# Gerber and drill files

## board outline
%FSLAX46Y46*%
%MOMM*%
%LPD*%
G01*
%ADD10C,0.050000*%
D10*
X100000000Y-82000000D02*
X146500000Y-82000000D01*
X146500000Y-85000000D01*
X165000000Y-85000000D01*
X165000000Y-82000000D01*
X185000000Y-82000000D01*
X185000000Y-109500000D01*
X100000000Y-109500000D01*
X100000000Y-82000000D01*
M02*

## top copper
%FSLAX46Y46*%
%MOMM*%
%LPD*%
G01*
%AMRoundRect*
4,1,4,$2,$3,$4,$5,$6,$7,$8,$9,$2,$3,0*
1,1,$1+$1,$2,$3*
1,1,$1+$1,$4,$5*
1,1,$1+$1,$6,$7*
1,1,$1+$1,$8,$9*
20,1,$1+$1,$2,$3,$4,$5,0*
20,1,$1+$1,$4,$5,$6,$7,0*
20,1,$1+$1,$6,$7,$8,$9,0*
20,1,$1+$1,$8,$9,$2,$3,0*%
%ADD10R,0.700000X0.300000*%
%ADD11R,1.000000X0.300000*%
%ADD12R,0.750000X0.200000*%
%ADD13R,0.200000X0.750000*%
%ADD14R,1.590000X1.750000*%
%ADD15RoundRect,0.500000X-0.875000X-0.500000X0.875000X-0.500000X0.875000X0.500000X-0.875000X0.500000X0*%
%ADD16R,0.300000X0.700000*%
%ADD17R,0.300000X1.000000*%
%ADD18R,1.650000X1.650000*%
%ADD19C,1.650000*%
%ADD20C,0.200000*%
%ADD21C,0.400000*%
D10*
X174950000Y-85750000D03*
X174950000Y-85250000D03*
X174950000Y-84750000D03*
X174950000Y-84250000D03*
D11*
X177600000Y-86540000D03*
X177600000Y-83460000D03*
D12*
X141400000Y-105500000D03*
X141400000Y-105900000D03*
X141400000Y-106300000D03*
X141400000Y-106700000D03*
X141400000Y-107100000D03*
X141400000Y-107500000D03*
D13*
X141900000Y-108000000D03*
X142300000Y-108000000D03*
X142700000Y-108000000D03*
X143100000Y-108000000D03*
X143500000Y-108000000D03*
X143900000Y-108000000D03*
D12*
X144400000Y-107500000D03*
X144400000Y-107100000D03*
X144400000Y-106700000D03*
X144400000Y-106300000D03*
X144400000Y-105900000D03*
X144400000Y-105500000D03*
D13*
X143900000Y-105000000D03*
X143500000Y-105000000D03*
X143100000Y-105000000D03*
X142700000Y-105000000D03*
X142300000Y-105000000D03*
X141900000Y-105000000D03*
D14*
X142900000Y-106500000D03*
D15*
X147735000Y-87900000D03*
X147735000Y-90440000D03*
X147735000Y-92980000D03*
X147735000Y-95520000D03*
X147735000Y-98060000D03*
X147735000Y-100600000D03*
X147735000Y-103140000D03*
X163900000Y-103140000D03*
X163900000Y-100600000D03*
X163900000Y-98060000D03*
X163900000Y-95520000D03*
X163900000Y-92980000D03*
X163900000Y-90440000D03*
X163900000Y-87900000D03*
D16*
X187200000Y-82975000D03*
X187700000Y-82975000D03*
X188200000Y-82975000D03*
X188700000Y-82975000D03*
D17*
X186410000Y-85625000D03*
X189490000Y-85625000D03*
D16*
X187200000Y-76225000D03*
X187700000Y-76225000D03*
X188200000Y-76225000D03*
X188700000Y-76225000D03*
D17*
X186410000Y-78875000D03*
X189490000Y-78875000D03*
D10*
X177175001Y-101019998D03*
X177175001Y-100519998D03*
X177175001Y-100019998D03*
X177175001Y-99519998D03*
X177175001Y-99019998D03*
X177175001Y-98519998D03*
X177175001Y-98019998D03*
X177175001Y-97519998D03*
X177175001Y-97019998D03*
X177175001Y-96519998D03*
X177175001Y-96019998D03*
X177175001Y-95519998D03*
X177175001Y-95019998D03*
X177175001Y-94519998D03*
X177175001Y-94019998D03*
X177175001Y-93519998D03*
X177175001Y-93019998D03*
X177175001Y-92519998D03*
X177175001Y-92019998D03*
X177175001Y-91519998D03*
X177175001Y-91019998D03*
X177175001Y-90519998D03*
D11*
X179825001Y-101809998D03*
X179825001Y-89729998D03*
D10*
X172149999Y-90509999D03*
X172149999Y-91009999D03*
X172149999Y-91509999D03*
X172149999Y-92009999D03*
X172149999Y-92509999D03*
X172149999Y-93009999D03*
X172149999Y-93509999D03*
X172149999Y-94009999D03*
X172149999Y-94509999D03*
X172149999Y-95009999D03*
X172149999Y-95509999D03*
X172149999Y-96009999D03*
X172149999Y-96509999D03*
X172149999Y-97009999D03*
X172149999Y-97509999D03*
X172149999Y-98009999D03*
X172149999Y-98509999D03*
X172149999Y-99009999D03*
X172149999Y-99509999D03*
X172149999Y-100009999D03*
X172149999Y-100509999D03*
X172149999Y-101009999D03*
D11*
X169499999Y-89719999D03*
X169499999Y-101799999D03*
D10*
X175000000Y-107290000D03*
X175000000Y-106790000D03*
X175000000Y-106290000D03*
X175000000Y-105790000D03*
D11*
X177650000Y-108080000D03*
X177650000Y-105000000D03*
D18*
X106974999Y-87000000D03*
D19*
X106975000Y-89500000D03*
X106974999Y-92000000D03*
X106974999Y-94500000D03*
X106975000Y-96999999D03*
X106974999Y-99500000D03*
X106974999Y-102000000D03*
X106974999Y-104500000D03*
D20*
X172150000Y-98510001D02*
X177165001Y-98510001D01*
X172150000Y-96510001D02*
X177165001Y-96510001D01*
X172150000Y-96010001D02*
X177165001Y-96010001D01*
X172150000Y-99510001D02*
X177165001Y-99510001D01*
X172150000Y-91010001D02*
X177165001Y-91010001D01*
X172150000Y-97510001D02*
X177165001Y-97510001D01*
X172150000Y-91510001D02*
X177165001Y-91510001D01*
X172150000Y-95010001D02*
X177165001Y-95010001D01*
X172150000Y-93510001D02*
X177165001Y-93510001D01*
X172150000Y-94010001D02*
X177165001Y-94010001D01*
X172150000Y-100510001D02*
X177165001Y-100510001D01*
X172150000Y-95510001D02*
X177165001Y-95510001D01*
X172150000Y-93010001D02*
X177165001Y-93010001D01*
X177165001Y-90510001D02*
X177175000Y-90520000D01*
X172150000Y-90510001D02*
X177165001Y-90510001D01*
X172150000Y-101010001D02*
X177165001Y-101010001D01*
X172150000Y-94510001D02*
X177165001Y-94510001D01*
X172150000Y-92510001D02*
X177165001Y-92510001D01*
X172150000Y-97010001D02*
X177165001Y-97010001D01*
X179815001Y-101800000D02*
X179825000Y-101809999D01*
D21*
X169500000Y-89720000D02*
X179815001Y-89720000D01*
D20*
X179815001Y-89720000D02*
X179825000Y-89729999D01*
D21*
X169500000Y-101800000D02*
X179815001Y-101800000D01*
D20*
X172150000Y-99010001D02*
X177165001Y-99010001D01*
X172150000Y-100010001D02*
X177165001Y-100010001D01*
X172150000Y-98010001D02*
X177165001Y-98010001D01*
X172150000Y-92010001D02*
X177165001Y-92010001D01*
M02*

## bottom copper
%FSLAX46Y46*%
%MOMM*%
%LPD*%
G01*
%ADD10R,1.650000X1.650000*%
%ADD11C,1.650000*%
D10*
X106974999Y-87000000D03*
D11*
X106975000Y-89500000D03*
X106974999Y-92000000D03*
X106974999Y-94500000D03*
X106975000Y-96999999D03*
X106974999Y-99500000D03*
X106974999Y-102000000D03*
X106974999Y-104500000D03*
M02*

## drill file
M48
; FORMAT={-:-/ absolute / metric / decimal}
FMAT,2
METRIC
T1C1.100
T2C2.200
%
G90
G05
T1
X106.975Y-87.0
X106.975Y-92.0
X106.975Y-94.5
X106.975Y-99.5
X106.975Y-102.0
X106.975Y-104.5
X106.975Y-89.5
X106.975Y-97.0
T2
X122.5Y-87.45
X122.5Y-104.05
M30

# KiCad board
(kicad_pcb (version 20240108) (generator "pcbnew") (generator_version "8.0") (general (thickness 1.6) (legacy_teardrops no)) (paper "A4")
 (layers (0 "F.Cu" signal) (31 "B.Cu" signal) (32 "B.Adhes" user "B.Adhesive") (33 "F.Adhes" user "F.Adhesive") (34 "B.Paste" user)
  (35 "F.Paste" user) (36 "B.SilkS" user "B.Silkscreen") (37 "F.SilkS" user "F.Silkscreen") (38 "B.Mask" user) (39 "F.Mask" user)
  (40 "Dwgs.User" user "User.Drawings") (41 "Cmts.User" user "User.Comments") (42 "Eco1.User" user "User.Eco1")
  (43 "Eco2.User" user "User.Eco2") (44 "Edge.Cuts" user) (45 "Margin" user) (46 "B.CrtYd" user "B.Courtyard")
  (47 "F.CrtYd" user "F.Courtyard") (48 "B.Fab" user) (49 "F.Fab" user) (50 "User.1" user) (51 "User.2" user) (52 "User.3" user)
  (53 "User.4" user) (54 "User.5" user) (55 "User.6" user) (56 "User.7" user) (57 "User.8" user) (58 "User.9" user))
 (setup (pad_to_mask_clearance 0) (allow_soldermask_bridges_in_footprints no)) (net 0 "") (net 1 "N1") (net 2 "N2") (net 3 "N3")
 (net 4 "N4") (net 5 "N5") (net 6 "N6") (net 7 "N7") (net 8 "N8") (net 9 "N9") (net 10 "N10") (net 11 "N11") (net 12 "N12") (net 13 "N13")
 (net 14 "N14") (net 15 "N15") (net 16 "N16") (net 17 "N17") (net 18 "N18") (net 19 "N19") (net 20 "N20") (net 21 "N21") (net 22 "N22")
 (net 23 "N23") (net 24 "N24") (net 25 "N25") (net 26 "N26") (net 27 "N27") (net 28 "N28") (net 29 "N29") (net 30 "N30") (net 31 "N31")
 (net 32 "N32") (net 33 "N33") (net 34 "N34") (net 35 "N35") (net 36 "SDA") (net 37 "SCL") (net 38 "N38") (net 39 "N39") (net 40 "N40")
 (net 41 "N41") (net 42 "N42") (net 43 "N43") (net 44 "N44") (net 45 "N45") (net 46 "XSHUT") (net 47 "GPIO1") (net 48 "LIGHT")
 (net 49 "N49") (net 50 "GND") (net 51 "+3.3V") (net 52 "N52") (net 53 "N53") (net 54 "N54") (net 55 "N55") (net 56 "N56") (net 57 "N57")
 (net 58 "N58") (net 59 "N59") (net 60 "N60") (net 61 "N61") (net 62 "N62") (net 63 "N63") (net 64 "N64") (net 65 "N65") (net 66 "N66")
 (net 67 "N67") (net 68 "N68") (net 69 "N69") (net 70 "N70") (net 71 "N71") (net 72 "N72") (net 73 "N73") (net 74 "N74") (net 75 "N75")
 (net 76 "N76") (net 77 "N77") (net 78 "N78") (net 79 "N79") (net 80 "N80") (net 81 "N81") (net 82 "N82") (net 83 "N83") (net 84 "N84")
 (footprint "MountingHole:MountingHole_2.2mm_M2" (layer "F.Cu") (at 122.5 104.05)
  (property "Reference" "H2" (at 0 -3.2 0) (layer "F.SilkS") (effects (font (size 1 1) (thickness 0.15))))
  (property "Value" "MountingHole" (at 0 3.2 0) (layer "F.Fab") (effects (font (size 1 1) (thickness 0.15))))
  (pad "" np_thru_hole circle (at 0 0) (size 2.2 2.2) (drill 2.2) (layers "*.Cu" "*.Mask")))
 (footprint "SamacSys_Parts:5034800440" (layer "F.Cu") (at 176.45 85 90)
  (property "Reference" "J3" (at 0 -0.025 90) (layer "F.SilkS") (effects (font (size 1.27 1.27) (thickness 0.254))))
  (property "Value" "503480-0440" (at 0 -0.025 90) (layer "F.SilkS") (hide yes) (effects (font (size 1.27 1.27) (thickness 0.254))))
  (pad "1" smd rect (at -0.75 -1.5 90) (size 0.3 0.7) (layers "F.Cu" "F.Paste" "F.Mask") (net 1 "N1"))
  (pad "2" smd rect (at -0.25 -1.5 90) (size 0.3 0.7) (layers "F.Cu" "F.Paste" "F.Mask") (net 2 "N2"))
  (pad "3" smd rect (at 0.25 -1.5 90) (size 0.3 0.7) (layers "F.Cu" "F.Paste" "F.Mask") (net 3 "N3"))
  (pad "4" smd rect (at 0.75 -1.5 90) (size 0.3 0.7) (layers "F.Cu" "F.Paste" "F.Mask") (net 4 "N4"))
  (pad "MP1" smd rect (at -1.54 1.15 90) (size 0.3 1) (layers "F.Cu" "F.Paste" "F.Mask") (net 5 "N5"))
  (pad "MP2" smd rect (at 1.54 1.15 90) (size 0.3 1) (layers "F.Cu" "F.Paste" "F.Mask") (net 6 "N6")))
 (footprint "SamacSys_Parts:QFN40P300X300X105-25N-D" (layer "F.Cu") (at 142.9 106.5)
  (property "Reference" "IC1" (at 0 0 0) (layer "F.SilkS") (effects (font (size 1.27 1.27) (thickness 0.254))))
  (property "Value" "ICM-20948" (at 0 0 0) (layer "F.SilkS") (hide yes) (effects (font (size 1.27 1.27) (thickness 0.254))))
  (pad "1" smd rect (at -1.5 -1 90) (size 0.2 0.75) (layers "F.Cu" "F.Paste" "F.Mask") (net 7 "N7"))
  (pad "2" smd rect (at -1.5 -0.6 90) (size 0.2 0.75) (layers "F.Cu" "F.Paste" "F.Mask") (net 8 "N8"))
  (pad "3" smd rect (at -1.5 -0.2 90) (size 0.2 0.75) (layers "F.Cu" "F.Paste" "F.Mask") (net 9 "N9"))
  (pad "4" smd rect (at -1.5 0.2 90) (size 0.2 0.75) (layers "F.Cu" "F.Paste" "F.Mask") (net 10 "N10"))
  (pad "5" smd rect (at -1.5 0.6 90) (size 0.2 0.75) (layers "F.Cu" "F.Paste" "F.Mask") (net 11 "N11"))
  (pad "6" smd rect (at -1.5 1 90) (size 0.2 0.75) (layers "F.Cu" "F.Paste" "F.Mask") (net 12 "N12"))
  (pad "7" smd rect (at -1 1.5) (size 0.2 0.75) (layers "F.Cu" "F.Paste" "F.Mask") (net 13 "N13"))
  (pad "8" smd rect (at -0.6 1.5) (size 0.2 0.75) (layers "F.Cu" "F.Paste" "F.Mask") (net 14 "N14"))
  (pad "9" smd rect (at -0.2 1.5) (size 0.2 0.75) (layers "F.Cu" "F.Paste" "F.Mask") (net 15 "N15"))
  (pad "10" smd rect (at 0.2 1.5) (size 0.2 0.75) (layers "F.Cu" "F.Paste" "F.Mask") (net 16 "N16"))
  (pad "11" smd rect (at 0.6 1.5) (size 0.2 0.75) (layers "F.Cu" "F.Paste" "F.Mask") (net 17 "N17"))
  (pad "12" smd rect (at 1 1.5) (size 0.2 0.75) (layers "F.Cu" "F.Paste" "F.Mask") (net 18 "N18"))
  (pad "13" smd rect (at 1.5 1 90) (size 0.2 0.75) (layers "F.Cu" "F.Paste" "F.Mask") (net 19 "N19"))
  (pad "14" smd rect (at 1.5 0.6 90) (size 0.2 0.75) (layers "F.Cu" "F.Paste" "F.Mask") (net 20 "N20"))
  (pad "15" smd rect (at 1.5 0.2 90) (size 0.2 0.75) (layers "F.Cu" "F.Paste" "F.Mask") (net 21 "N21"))
  (pad "16" smd rect (at 1.5 -0.2 90) (size 0.2 0.75) (layers "F.Cu" "F.Paste" "F.Mask") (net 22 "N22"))
  (pad "17" smd rect (at 1.5 -0.6 90) (size 0.2 0.75) (layers "F.Cu" "F.Paste" "F.Mask") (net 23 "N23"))
  (pad "18" smd rect (at 1.5 -1 90) (size 0.2 0.75) (layers "F.Cu" "F.Paste" "F.Mask") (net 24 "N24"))
  (pad "19" smd rect (at 1 -1.5) (size 0.2 0.75) (layers "F.Cu" "F.Paste" "F.Mask") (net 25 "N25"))
  (pad "20" smd rect (at 0.6 -1.5) (size 0.2 0.75) (layers "F.Cu" "F.Paste" "F.Mask") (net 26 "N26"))
  (pad "21" smd rect (at 0.2 -1.5) (size 0.2 0.75) (layers "F.Cu" "F.Paste" "F.Mask") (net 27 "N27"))
  (pad "22" smd rect (at -0.2 -1.5) (size 0.2 0.75) (layers "F.Cu" "F.Paste" "F.Mask") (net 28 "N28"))
  (pad "23" smd rect (at -0.6 -1.5) (size 0.2 0.75) (layers "F.Cu" "F.Paste" "F.Mask") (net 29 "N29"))
  (pad "24" smd rect (at -1 -1.5) (size 0.2 0.75) (layers "F.Cu" "F.Paste" "F.Mask") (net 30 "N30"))
  (pad "25" smd rect (at 0 0) (size 1.59 1.75) (layers "F.Cu" "F.Paste" "F.Mask") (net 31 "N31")))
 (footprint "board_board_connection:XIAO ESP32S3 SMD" (layer "F.Cu") (at 155.796364 95.473)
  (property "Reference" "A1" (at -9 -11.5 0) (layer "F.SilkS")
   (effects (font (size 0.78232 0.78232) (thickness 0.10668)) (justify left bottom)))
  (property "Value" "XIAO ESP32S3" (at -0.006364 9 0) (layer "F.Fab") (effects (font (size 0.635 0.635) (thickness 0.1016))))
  (pad "1" smd roundrect (at -8.061364 -7.573) (size 2.75 2) (layers "F.Cu" "F.Paste" "F.Mask") (roundrect_rratio 0.25) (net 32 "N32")
   (solder_mask_margin 0.0508) (thermal_bridge_angle 45))
  (pad "2" smd roundrect (at -8.061364 -5.033) (size 2.75 2) (layers "F.Cu" "F.Paste" "F.Mask") (roundrect_rratio 0.25) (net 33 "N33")
   (solder_mask_margin 0.0508) (thermal_bridge_angle 45))
  (pad "3" smd roundrect (at -8.061364 -2.493) (size 2.75 2) (layers "F.Cu" "F.Paste" "F.Mask") (roundrect_rratio 0.25) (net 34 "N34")
   (solder_mask_margin 0.0508) (thermal_bridge_angle 45))
  (pad "4" smd roundrect (at -8.061364 0.047) (size 2.75 2) (layers "F.Cu" "F.Paste" "F.Mask") (roundrect_rratio 0.25) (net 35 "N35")
   (solder_mask_margin 0.0508) (thermal_bridge_angle 45))
  (pad "5" smd roundrect (at -8.061364 2.587) (size 2.75 2) (layers "F.Cu" "F.Paste" "F.Mask") (roundrect_rratio 0.25) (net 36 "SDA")
   (solder_mask_margin 0.0508) (thermal_bridge_angle 45))
  (pad "6" smd roundrect (at -8.061364 5.127) (size 2.75 2) (layers "F.Cu" "F.Paste" "F.Mask") (roundrect_rratio 0.25) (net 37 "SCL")
   (solder_mask_margin 0.0508) (thermal_bridge_angle 45))
  (pad "7" smd roundrect (at -8.061364 7.667) (size 2.75 2) (layers "F.Cu" "F.Paste" "F.Mask") (roundrect_rratio 0.25) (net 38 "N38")
   (solder_mask_margin 0.0508) (thermal_bridge_angle 45))
  (pad "8" smd roundrect (at 8.103636 7.667) (size 2.75 2) (layers "F.Cu" "F.Paste" "F.Mask") (roundrect_rratio 0.25) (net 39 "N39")
   (solder_mask_margin 0.0508) (thermal_bridge_angle 45))
  (pad "9" smd roundrect (at 8.103636 5.127) (size 2.75 2) (layers "F.Cu" "F.Paste" "F.Mask") (roundrect_rratio 0.25) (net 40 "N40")
   (solder_mask_margin 0.0508) (thermal_bridge_angle 45))
  (pad "10" smd roundrect (at 8.103636 2.587) (size 2.75 2) (layers "F.Cu" "F.Paste" "F.Mask") (roundrect_rratio 0.25) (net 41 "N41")
   (solder_mask_margin 0.0508) (thermal_bridge_angle 45))
  (pad "11" smd roundrect (at 8.103636 0.047) (size 2.75 2) (layers "F.Cu" "F.Paste" "F.Mask") (roundrect_rratio 0.25) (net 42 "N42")
   (solder_mask_margin 0.0508) (thermal_bridge_angle 45))
  (pad "12" smd roundrect (at 8.103636 -2.493) (size 2.75 2) (layers "F.Cu" "F.Paste" "F.Mask") (roundrect_rratio 0.25) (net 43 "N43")
   (solder_mask_margin 0.0508) (thermal_bridge_angle 45))
  (pad "13" smd roundrect (at 8.103636 -5.033) (size 2.75 2) (layers "F.Cu" "F.Paste" "F.Mask") (roundrect_rratio 0.25) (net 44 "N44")
   (solder_mask_margin 0.0508) (thermal_bridge_angle 45))
  (pad "14" smd roundrect (at 8.103636 -7.573) (size 2.75 2) (layers "F.Cu" "F.Paste" "F.Mask") (roundrect_rratio 0.25) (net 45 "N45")
   (solder_mask_margin 0.0508) (thermal_bridge_angle 45)))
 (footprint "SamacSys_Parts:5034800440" (layer "F.Cu") (at 187.95 84.475)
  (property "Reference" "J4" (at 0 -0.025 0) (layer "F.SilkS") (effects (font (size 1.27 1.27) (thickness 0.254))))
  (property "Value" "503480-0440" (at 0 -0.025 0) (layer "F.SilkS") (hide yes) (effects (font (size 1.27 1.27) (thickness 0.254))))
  (pad "1" smd rect (at -0.75 -1.5) (size 0.3 0.7) (layers "F.Cu" "F.Paste" "F.Mask") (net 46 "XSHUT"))
  (pad "2" smd rect (at -0.25 -1.5) (size 0.3 0.7) (layers "F.Cu" "F.Paste" "F.Mask") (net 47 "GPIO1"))
  (pad "3" smd rect (at 0.25 -1.5) (size 0.3 0.7) (layers "F.Cu" "F.Paste" "F.Mask") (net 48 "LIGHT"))
  (pad "4" smd rect (at 0.75 -1.5) (size 0.3 0.7) (layers "F.Cu" "F.Paste" "F.Mask") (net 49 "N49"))
  (pad "MP1" smd rect (at -1.54 1.15) (size 0.3 1) (layers "F.Cu" "F.Paste" "F.Mask") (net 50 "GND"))
  (pad "MP2" smd rect (at 1.54 1.15) (size 0.3 1) (layers "F.Cu" "F.Paste" "F.Mask") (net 50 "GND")))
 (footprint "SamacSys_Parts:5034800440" (layer "F.Cu") (at 187.95 77.725)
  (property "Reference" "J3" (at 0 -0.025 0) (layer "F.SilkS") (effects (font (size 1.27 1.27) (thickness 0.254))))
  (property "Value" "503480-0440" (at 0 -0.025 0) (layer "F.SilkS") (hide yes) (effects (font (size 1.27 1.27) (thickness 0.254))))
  (pad "1" smd rect (at -0.75 -1.5) (size 0.3 0.7) (layers "F.Cu" "F.Paste" "F.Mask") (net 36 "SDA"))
  (pad "2" smd rect (at -0.25 -1.5) (size 0.3 0.7) (layers "F.Cu" "F.Paste" "F.Mask") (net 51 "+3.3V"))
  (pad "3" smd rect (at 0.25 -1.5) (size 0.3 0.7) (layers "F.Cu" "F.Paste" "F.Mask") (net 37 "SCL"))
  (pad "4" smd rect (at 0.75 -1.5) (size 0.3 0.7) (layers "F.Cu" "F.Paste" "F.Mask") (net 50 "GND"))
  (pad "MP1" smd rect (at -1.54 1.15) (size 0.3 1) (layers "F.Cu" "F.Paste" "F.Mask") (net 50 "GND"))
  (pad "MP2" smd rect (at 1.54 1.15) (size 0.3 1) (layers "F.Cu" "F.Paste" "F.Mask") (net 50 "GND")))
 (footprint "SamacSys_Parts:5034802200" (layer "F.Cu") (at 176.925001 95.769998 90)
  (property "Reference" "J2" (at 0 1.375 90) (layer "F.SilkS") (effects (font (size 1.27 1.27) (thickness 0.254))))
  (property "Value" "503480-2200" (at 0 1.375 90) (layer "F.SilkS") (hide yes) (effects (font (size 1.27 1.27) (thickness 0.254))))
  (pad "1" smd rect (at -5.25 0.25 90) (size 0.3 0.7) (layers "F.Cu" "F.Paste" "F.Mask") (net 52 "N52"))
  (pad "2" smd rect (at -4.75 0.25 90) (size 0.3 0.7) (layers "F.Cu" "F.Paste" "F.Mask") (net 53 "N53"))
  (pad "3" smd rect (at -4.25 0.25 90) (size 0.3 0.7) (layers "F.Cu" "F.Paste" "F.Mask") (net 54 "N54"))
  (pad "4" smd rect (at -3.75 0.25 90) (size 0.3 0.7) (layers "F.Cu" "F.Paste" "F.Mask") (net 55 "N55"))
  (pad "5" smd rect (at -3.25 0.25 90) (size 0.3 0.7) (layers "F.Cu" "F.Paste" "F.Mask") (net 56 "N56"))
  (pad "6" smd rect (at -2.75 0.25 90) (size 0.3 0.7) (layers "F.Cu" "F.Paste" "F.Mask") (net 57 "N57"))
  (pad "7" smd rect (at -2.25 0.25 90) (size 0.3 0.7) (layers "F.Cu" "F.Paste" "F.Mask") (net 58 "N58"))
  (pad "8" smd rect (at -1.75 0.25 90) (size 0.3 0.7) (layers "F.Cu" "F.Paste" "F.Mask") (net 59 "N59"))
  (pad "9" smd rect (at -1.25 0.25 90) (size 0.3 0.7) (layers "F.Cu" "F.Paste" "F.Mask") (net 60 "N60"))
  (pad "10" smd rect (at -0.75 0.25 90) (size 0.3 0.7) (layers "F.Cu" "F.Paste" "F.Mask") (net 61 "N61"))
  (pad "11" smd rect (at -0.25 0.25 90) (size 0.3 0.7) (layers "F.Cu" "F.Paste" "F.Mask") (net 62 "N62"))
  (pad "12" smd rect (at 0.25 0.25 90) (size 0.3 0.7) (layers "F.Cu" "F.Paste" "F.Mask") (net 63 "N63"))
  (pad "13" smd rect (at 0.75 0.25 90) (size 0.3 0.7) (layers "F.Cu" "F.Paste" "F.Mask") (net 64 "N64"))
  (pad "14" smd rect (at 1.25 0.25 90) (size 0.3 0.7) (layers "F.Cu" "F.Paste" "F.Mask") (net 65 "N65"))
  (pad "15" smd rect (at 1.75 0.25 90) (size 0.3 0.7) (layers "F.Cu" "F.Paste" "F.Mask") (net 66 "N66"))
  (pad "16" smd rect (at 2.25 0.25 90) (size 0.3 0.7) (layers "F.Cu" "F.Paste" "F.Mask") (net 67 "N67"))
  (pad "17" smd rect (at 2.75 0.25 90) (size 0.3 0.7) (layers "F.Cu" "F.Paste" "F.Mask") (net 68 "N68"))
  (pad "18" smd rect (at 3.25 0.25 90) (size 0.3 0.7) (layers "F.Cu" "F.Paste" "F.Mask") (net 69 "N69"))
  (pad "19" smd rect (at 3.75 0.25 90) (size 0.3 0.7) (layers "F.Cu" "F.Paste" "F.Mask") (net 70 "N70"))
  (pad "20" smd rect (at 4.25 0.25 90) (size 0.3 0.7) (layers "F.Cu" "F.Paste" "F.Mask") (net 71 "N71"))
  (pad "21" smd rect (at 4.75 0.25 90) (size 0.3 0.7) (layers "F.Cu" "F.Paste" "F.Mask") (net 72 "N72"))
  (pad "22" smd rect (at 5.25 0.25 90) (size 0.3 0.7) (layers "F.Cu" "F.Paste" "F.Mask") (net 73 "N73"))
  (pad "MP1" smd rect (at -6.04 2.9 90) (size 0.3 1) (layers "F.Cu" "F.Paste" "F.Mask") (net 50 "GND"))
  (pad "MP2" smd rect (at 6.04 2.9 90) (size 0.3 1) (layers "F.Cu" "F.Paste" "F.Mask") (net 50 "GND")))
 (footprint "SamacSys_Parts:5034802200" (layer "F.Cu") (at 172.399999 95.759999 -90)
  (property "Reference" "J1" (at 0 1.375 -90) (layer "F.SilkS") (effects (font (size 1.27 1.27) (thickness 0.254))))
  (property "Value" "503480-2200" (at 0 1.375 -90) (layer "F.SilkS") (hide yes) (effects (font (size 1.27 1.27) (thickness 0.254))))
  (pad "1" smd rect (at -5.25 0.25 270) (size 0.3 0.7) (layers "F.Cu" "F.Paste" "F.Mask") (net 73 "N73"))
  (pad "2" smd rect (at -4.75 0.25 270) (size 0.3 0.7) (layers "F.Cu" "F.Paste" "F.Mask") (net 72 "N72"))
  (pad "3" smd rect (at -4.25 0.25 270) (size 0.3 0.7) (layers "F.Cu" "F.Paste" "F.Mask") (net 71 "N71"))
  (pad "4" smd rect (at -3.75 0.25 270) (size 0.3 0.7) (layers "F.Cu" "F.Paste" "F.Mask") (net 70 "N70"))
  (pad "5" smd rect (at -3.25 0.25 270) (size 0.3 0.7) (layers "F.Cu" "F.Paste" "F.Mask") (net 69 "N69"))
  (pad "6" smd rect (at -2.75 0.25 270) (size 0.3 0.7) (layers "F.Cu" "F.Paste" "F.Mask") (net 68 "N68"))
  (pad "7" smd rect (at -2.25 0.25 270) (size 0.3 0.7) (layers "F.Cu" "F.Paste" "F.Mask") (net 67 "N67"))
  (pad "8" smd rect (at -1.75 0.25 270) (size 0.3 0.7) (layers "F.Cu" "F.Paste" "F.Mask") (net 66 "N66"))
  (pad "9" smd rect (at -1.25 0.25 270) (size 0.3 0.7) (layers "F.Cu" "F.Paste" "F.Mask") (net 65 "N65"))
  (pad "10" smd rect (at -0.75 0.25 270) (size 0.3 0.7) (layers "F.Cu" "F.Paste" "F.Mask") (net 64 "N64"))
  (pad "11" smd rect (at -0.25 0.25 270) (size 0.3 0.7) (layers "F.Cu" "F.Paste" "F.Mask") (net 63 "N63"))
  (pad "12" smd rect (at 0.25 0.25 270) (size 0.3 0.7) (layers "F.Cu" "F.Paste" "F.Mask") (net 62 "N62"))
  (pad "13" smd rect (at 0.75 0.25 270) (size 0.3 0.7) (layers "F.Cu" "F.Paste" "F.Mask") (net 61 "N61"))
  (pad "14" smd rect (at 1.25 0.25 270) (size 0.3 0.7) (layers "F.Cu" "F.Paste" "F.Mask") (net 60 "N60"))
  (pad "15" smd rect (at 1.75 0.25 270) (size 0.3 0.7) (layers "F.Cu" "F.Paste" "F.Mask") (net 59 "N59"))
  (pad "16" smd rect (at 2.25 0.25 270) (size 0.3 0.7) (layers "F.Cu" "F.Paste" "F.Mask") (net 58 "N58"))
  (pad "17" smd rect (at 2.75 0.25 270) (size 0.3 0.7) (layers "F.Cu" "F.Paste" "F.Mask") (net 57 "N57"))
  (pad "18" smd rect (at 3.25 0.25 270) (size 0.3 0.7) (layers "F.Cu" "F.Paste" "F.Mask") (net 56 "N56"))
  (pad "19" smd rect (at 3.75 0.25 270) (size 0.3 0.7) (layers "F.Cu" "F.Paste" "F.Mask") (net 55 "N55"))
  (pad "20" smd rect (at 4.25 0.25 270) (size 0.3 0.7) (layers "F.Cu" "F.Paste" "F.Mask") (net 54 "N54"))
  (pad "21" smd rect (at 4.75 0.25 270) (size 0.3 0.7) (layers "F.Cu" "F.Paste" "F.Mask") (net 53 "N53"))
  (pad "22" smd rect (at 5.25 0.25 270) (size 0.3 0.7) (layers "F.Cu" "F.Paste" "F.Mask") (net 52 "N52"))
  (pad "MP1" smd rect (at -6.04 2.9 270) (size 0.3 1) (layers "F.Cu" "F.Paste" "F.Mask") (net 50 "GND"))
  (pad "MP2" smd rect (at 6.04 2.9 270) (size 0.3 1) (layers "F.Cu" "F.Paste" "F.Mask") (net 50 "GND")))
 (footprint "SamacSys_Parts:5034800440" (layer "F.Cu") (at 176.5 106.54 90)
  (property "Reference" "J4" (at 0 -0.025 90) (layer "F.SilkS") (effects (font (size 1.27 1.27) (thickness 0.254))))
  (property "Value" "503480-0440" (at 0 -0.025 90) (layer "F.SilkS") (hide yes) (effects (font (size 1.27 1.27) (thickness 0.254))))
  (pad "1" smd rect (at -0.75 -1.5 90) (size 0.3 0.7) (layers "F.Cu" "F.Paste" "F.Mask") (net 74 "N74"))
  (pad "2" smd rect (at -0.25 -1.5 90) (size 0.3 0.7) (layers "F.Cu" "F.Paste" "F.Mask") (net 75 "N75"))
  (pad "3" smd rect (at 0.25 -1.5 90) (size 0.3 0.7) (layers "F.Cu" "F.Paste" "F.Mask") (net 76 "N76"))
  (pad "4" smd rect (at 0.75 -1.5 90) (size 0.3 0.7) (layers "F.Cu" "F.Paste" "F.Mask") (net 49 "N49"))
  (pad "MP1" smd rect (at -1.54 1.15 90) (size 0.3 1) (layers "F.Cu" "F.Paste" "F.Mask") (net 6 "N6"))
  (pad "MP2" smd rect (at 1.54 1.15 90) (size 0.3 1) (layers "F.Cu" "F.Paste" "F.Mask") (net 50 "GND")))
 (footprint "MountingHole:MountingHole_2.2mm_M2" (layer "F.Cu") (at 122.5 87.45)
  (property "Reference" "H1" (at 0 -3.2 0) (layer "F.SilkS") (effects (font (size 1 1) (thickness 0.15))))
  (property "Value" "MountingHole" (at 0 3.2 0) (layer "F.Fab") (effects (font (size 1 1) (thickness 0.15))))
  (pad "" np_thru_hole circle (at 0 0) (size 2.2 2.2) (drill 2.2) (layers "*.Cu" "*.Mask")))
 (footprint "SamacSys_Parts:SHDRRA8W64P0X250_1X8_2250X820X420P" (layer "B.Cu") (at 106.974999 87 -90)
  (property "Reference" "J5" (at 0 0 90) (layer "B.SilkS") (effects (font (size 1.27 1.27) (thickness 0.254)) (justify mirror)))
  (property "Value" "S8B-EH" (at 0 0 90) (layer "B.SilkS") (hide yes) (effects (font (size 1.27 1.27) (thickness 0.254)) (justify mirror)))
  (pad "1" thru_hole rect (at 0 0 270) (size 1.65 1.65) (drill 1.1) (layers "*.Cu" "*.Mask") (remove_unused_layers no) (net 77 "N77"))
  (pad "2" thru_hole circle (at 2.5 -0.000001 270) (size 1.65 1.65) (drill 1.1) (layers "*.Cu" "*.Mask") (remove_unused_layers no)
   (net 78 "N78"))
  (pad "3" thru_hole circle (at 5 0 270) (size 1.65 1.65) (drill 1.1) (layers "*.Cu" "*.Mask") (remove_unused_layers no) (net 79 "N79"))
  (pad "4" thru_hole circle (at 7.5 0 270) (size 1.65 1.65) (drill 1.1) (layers "*.Cu" "*.Mask") (remove_unused_layers no) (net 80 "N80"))
  (pad "5" thru_hole circle (at 9.999999 -0.000001 270) (size 1.65 1.65) (drill 1.1) (layers "*.Cu" "*.Mask") (remove_unused_layers no)
   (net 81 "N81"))
  (pad "6" thru_hole circle (at 12.5 0 270) (size 1.65 1.65) (drill 1.1) (layers "*.Cu" "*.Mask") (remove_unused_layers no) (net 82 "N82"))
  (pad "7" thru_hole circle (at 15 0 270) (size 1.65 1.65) (drill 1.1) (layers "*.Cu" "*.Mask") (remove_unused_layers no) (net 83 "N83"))
  (pad "8" thru_hole circle (at 17.5 0 270) (size 1.65 1.65) (drill 1.1) (layers "*.Cu" "*.Mask") (remove_unused_layers no) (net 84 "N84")))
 (gr_poly
  (pts (xy 100 82) (xy 146.5 82) (xy 146.5 85) (xy 165 85) (xy 165 82) (xy 185 82) (xy 185 109.5) (xy 100 109.5))
  (stroke (width 0.05) (type solid)) (fill none) (layer "Edge.Cuts"))
 (segment (start 172.15 98.510001) (end 177.165001 98.510001) (width 0.2) (layer "F.Cu") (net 57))
 (segment (start 172.15 96.510001) (end 177.165001 96.510001) (width 0.2) (layer "F.Cu") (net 61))
 (segment (start 172.15 96.010001) (end 177.165001 96.010001) (width 0.2) (layer "F.Cu") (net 62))
 (segment (start 172.15 99.510001) (end 177.165001 99.510001) (width 0.2) (layer "F.Cu") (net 55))
 (segment (start 172.15 91.010001) (end 177.165001 91.010001) (width 0.2) (layer "F.Cu") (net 72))
 (segment (start 172.15 97.510001) (end 177.165001 97.510001) (width 0.2) (layer "F.Cu") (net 59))
 (segment (start 172.15 91.510001) (end 177.165001 91.510001) (width 0.2) (layer "F.Cu") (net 71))
 (segment (start 172.15 95.010001) (end 177.165001 95.010001) (width 0.2) (layer "F.Cu") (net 64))
 (segment (start 172.15 93.510001) (end 177.165001 93.510001) (width 0.2) (layer "F.Cu") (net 67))
 (segment (start 172.15 94.010001) (end 177.165001 94.010001) (width 0.2) (layer "F.Cu") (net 66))
 (segment (start 172.15 100.510001) (end 177.165001 100.510001) (width 0.2) (layer "F.Cu") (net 53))
 (segment (start 172.15 95.510001) (end 177.165001 95.510001) (width 0.2) (layer "F.Cu") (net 63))
 (segment (start 172.15 93.010001) (end 177.165001 93.010001) (width 0.2) (layer "F.Cu") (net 68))
 (segment (start 177.165001 90.510001) (end 177.175 90.52) (width 0.2) (layer "F.Cu") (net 73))
 (segment (start 172.15 90.510001) (end 177.165001 90.510001) (width 0.2) (layer "F.Cu") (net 73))
 (segment (start 172.15 101.010001) (end 177.165001 101.010001) (width 0.2) (layer "F.Cu") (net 52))
 (segment (start 172.15 94.510001) (end 177.165001 94.510001) (width 0.2) (layer "F.Cu") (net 65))
 (segment (start 172.15 92.510001) (end 177.165001 92.510001) (width 0.2) (layer "F.Cu") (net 69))
 (segment (start 172.15 97.010001) (end 177.165001 97.010001) (width 0.2) (layer "F.Cu") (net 60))
 (segment (start 179.815001 101.8) (end 179.825 101.809999) (width 0.2) (layer "F.Cu") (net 50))
 (segment (start 169.5 89.72) (end 179.815001 89.72) (width 0.4) (layer "F.Cu") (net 50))
 (segment (start 179.815001 89.72) (end 179.825 89.729999) (width 0.2) (layer "F.Cu") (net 50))
 (segment (start 169.5 101.8) (end 179.815001 101.8) (width 0.4) (layer "F.Cu") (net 50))
 (segment (start 172.15 99.010001) (end 177.165001 99.010001) (width 0.2) (layer "F.Cu") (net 56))
 (segment (start 172.15 100.010001) (end 177.165001 100.010001) (width 0.2) (layer "F.Cu") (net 54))
 (segment (start 172.15 98.010001) (end 177.165001 98.010001) (width 0.2) (layer "F.Cu") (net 58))
 (segment (start 172.15 92.010001) (end 177.165001 92.010001) (width 0.2) (layer "F.Cu") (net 70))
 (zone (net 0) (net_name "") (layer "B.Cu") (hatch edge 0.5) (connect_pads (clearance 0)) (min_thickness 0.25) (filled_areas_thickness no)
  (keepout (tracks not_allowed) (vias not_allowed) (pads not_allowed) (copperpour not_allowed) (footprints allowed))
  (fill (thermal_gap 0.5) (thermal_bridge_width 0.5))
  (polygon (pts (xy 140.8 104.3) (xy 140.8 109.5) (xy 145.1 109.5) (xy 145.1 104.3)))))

